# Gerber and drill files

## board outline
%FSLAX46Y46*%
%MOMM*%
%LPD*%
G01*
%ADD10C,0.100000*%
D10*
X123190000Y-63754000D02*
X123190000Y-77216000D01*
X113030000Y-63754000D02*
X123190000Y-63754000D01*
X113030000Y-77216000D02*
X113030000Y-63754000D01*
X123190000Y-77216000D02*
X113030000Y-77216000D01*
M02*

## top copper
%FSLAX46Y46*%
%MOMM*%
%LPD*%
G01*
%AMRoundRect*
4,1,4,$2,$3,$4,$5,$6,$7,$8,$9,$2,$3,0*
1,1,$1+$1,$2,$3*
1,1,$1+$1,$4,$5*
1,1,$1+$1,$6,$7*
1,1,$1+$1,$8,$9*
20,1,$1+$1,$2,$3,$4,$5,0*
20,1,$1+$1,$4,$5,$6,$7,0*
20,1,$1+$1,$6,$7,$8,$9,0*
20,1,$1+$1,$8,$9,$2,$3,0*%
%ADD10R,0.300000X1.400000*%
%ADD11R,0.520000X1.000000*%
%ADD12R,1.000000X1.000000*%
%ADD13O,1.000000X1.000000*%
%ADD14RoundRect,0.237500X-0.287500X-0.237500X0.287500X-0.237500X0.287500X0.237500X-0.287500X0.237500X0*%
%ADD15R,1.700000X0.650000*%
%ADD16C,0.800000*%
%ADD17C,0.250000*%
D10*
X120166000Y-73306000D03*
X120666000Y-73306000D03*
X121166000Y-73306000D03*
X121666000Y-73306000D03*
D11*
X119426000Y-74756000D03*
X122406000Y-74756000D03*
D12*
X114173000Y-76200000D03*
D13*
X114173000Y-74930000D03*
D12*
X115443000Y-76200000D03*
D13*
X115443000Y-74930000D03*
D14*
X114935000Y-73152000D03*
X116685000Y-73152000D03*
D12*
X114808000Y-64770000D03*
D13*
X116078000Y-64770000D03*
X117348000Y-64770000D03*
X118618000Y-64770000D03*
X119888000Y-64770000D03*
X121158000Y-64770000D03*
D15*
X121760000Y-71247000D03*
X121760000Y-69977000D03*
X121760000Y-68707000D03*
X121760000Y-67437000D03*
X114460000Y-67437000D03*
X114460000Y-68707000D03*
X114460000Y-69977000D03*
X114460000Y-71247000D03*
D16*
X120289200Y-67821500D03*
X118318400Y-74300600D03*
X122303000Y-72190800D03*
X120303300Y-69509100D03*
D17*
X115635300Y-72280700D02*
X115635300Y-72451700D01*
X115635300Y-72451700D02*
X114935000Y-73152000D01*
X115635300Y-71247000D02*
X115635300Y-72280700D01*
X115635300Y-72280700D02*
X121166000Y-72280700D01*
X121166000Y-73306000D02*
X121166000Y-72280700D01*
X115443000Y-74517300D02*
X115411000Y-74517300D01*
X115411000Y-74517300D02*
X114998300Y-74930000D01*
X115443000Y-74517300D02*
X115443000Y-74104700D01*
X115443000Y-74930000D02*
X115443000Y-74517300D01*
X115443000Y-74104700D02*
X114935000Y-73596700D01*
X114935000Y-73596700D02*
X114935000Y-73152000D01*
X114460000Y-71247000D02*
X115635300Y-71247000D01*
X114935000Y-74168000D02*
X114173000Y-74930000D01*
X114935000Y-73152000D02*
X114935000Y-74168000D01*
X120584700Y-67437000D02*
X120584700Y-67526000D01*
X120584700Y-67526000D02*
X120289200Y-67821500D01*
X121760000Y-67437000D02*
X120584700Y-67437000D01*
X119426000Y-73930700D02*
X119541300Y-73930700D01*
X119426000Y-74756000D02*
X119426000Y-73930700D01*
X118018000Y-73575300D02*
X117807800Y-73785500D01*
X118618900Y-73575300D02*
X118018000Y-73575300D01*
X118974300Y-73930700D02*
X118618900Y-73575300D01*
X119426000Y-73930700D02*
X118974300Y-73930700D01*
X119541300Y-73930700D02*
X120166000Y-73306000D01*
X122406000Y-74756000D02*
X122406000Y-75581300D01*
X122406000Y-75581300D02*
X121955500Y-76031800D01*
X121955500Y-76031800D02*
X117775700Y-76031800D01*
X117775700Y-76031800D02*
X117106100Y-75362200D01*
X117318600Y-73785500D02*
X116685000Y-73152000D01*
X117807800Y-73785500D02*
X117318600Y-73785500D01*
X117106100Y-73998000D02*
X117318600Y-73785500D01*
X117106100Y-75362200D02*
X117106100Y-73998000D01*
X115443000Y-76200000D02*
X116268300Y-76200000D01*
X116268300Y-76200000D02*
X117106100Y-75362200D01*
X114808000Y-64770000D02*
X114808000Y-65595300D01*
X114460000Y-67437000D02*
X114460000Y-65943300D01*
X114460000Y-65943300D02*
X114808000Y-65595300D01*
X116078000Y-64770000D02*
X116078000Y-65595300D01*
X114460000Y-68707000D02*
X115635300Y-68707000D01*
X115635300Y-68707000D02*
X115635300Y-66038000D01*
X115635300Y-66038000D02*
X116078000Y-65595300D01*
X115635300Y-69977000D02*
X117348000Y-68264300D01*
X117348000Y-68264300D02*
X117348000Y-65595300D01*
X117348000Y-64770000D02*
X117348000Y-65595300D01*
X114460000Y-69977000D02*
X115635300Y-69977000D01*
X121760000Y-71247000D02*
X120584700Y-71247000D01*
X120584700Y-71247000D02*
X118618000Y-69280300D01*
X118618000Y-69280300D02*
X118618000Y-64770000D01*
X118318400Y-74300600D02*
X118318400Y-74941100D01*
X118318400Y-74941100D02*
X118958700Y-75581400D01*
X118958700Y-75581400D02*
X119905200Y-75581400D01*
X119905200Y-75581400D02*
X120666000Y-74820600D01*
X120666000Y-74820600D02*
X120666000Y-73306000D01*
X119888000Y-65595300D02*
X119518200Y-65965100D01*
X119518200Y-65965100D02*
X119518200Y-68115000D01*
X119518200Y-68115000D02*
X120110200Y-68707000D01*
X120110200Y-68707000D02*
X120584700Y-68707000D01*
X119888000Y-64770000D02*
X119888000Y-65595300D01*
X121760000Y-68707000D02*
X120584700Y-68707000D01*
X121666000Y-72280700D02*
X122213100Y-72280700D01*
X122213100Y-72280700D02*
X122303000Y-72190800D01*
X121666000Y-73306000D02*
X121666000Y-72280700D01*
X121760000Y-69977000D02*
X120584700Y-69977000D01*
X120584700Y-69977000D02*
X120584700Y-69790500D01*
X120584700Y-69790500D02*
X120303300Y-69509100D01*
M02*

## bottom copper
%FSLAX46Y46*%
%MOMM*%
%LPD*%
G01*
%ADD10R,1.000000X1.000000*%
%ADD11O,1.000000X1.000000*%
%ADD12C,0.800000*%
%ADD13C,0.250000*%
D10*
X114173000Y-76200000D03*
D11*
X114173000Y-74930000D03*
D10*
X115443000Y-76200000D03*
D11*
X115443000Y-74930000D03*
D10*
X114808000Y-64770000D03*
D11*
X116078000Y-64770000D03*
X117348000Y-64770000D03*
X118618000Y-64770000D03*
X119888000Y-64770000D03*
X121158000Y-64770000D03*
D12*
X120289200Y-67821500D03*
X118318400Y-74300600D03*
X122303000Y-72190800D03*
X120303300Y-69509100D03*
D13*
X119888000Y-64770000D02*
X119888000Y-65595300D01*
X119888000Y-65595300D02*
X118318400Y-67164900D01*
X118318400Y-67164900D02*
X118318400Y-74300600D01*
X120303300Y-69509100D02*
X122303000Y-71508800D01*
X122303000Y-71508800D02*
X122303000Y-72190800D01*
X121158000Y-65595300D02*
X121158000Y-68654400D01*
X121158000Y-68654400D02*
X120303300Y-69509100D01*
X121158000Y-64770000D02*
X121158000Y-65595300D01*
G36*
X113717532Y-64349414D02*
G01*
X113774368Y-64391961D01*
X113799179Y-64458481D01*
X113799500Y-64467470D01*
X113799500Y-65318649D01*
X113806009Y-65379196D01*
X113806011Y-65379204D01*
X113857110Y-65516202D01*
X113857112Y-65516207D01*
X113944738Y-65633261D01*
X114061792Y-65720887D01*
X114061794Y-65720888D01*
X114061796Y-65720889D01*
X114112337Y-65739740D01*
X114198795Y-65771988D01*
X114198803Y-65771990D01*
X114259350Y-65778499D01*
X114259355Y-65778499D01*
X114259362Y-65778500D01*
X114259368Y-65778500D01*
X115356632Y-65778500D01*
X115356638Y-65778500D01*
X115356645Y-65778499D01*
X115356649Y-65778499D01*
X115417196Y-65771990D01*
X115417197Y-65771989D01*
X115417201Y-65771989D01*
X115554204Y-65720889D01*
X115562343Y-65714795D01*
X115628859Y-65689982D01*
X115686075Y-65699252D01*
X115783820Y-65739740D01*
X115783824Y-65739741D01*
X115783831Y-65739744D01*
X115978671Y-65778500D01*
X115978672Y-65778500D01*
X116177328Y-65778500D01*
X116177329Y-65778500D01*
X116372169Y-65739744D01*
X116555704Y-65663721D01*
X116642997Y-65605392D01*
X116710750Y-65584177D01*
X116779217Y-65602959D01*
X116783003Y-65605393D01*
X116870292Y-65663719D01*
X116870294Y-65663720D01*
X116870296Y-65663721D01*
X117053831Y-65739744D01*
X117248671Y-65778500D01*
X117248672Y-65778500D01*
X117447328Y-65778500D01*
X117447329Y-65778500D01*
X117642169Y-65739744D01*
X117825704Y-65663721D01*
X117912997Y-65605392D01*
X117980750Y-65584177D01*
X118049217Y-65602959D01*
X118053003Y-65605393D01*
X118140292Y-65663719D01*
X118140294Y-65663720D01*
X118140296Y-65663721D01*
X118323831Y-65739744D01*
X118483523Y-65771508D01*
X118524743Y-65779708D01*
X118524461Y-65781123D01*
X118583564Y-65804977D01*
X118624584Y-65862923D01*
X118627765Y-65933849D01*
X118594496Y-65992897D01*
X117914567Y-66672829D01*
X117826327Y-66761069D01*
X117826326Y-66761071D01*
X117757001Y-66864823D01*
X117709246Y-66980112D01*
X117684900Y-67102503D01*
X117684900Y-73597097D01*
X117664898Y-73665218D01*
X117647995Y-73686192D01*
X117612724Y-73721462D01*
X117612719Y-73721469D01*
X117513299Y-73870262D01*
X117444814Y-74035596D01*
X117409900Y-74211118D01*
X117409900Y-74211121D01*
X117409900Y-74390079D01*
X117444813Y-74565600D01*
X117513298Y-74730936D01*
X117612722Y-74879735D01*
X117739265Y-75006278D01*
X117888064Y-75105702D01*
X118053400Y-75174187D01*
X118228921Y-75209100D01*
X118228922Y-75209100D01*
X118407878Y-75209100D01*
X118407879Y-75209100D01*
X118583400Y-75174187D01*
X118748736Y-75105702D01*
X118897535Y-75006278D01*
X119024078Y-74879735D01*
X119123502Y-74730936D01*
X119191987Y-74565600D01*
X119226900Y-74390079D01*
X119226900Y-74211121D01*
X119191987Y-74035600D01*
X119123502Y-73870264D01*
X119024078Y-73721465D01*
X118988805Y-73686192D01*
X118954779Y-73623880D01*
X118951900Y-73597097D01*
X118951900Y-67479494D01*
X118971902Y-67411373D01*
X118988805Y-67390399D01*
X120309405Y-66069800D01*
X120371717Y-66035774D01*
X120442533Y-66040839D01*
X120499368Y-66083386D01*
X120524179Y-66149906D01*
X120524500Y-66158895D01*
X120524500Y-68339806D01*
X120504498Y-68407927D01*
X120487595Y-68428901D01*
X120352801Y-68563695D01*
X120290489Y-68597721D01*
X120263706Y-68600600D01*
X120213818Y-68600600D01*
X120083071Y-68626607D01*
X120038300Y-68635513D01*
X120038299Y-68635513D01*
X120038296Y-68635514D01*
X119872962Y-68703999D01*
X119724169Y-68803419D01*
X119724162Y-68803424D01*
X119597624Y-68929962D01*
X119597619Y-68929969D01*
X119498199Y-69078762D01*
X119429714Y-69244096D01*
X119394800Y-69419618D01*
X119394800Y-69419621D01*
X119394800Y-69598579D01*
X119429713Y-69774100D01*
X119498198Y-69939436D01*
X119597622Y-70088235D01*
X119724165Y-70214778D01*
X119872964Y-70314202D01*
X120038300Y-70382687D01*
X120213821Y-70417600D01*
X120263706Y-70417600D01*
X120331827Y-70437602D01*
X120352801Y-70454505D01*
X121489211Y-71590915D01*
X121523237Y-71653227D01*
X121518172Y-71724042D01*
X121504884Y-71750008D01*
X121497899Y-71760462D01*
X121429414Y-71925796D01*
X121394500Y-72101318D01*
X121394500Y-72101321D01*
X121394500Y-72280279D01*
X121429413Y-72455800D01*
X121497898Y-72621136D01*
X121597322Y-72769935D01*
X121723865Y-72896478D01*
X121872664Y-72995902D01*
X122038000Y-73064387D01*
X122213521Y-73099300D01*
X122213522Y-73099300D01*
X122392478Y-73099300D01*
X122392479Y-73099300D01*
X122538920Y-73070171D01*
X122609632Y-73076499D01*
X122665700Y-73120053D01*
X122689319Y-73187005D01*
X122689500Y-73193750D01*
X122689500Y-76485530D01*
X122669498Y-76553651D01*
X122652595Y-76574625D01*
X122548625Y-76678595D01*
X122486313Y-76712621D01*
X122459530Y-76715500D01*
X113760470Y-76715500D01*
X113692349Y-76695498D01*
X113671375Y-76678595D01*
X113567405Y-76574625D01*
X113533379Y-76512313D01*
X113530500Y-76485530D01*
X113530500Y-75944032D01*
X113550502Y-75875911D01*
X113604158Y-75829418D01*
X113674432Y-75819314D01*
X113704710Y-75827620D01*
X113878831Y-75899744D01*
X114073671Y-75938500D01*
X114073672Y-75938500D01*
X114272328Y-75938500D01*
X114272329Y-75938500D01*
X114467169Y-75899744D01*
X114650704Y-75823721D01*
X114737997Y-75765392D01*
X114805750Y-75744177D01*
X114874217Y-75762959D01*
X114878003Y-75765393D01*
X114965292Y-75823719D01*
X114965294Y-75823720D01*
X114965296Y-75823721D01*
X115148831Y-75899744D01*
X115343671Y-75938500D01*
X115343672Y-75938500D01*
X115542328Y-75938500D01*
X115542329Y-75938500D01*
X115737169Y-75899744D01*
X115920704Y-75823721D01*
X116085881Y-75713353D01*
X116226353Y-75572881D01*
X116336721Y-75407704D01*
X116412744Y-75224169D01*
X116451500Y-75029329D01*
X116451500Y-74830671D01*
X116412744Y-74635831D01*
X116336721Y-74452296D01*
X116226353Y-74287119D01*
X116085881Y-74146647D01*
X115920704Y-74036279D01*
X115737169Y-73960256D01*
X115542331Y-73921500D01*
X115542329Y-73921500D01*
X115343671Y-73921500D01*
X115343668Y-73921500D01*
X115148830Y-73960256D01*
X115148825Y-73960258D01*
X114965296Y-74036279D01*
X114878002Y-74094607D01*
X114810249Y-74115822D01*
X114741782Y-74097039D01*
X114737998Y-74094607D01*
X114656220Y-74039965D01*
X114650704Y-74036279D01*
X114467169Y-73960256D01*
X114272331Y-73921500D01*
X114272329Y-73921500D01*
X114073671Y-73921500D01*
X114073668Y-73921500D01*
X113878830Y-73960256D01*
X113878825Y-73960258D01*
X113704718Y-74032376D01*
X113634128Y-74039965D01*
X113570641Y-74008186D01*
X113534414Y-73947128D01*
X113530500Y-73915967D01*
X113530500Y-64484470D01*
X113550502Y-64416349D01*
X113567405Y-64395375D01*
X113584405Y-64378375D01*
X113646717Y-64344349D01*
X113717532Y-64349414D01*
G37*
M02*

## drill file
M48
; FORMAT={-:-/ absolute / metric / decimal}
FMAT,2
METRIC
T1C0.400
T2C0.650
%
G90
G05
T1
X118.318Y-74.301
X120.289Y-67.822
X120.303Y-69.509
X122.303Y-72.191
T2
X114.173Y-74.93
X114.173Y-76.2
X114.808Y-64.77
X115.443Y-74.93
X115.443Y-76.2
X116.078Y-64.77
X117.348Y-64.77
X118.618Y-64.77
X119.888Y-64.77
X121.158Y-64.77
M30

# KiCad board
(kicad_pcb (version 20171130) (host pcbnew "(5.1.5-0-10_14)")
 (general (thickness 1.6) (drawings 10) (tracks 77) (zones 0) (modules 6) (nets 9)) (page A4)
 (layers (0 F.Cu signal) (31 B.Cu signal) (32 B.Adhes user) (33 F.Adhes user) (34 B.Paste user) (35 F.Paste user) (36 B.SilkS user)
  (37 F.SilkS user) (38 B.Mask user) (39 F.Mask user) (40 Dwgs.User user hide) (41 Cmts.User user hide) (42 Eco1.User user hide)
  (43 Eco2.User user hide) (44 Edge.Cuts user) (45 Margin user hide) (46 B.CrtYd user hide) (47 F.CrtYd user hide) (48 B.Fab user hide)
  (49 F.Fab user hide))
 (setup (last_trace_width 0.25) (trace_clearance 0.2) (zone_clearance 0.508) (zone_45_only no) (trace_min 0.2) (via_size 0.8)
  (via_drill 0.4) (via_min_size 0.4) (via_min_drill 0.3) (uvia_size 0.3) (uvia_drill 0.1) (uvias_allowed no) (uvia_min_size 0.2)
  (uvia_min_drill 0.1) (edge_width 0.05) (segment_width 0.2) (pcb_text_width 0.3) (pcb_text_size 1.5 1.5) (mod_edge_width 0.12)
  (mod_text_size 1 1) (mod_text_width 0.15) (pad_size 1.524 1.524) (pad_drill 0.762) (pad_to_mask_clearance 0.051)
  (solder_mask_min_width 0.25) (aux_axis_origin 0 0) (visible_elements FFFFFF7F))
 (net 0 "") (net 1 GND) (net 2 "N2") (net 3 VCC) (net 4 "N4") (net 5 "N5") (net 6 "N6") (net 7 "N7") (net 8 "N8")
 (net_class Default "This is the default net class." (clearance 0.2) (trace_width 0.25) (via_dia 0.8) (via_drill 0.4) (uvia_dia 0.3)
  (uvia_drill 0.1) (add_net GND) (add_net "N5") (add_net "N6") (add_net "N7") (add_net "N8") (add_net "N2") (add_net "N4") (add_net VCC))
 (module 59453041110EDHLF (layer F.Cu) (at 120.916 73.406)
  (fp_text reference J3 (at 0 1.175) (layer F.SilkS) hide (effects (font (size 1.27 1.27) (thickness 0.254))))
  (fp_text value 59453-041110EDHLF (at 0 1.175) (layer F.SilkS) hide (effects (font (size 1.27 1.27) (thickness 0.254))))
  (pad 1 smd rect (at -0.75 -0.1) (size 0.3 1.4) (layers F.Cu F.Paste F.Mask) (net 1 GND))
  (pad 2 smd rect (at -0.25 -0.1) (size 0.3 1.4) (layers F.Cu F.Paste F.Mask) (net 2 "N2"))
  (pad 3 smd rect (at 0.25 -0.1) (size 0.3 1.4) (layers F.Cu F.Paste F.Mask) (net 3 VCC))
  (pad 4 smd rect (at 0.75 -0.1) (size 0.3 1.4) (layers F.Cu F.Paste F.Mask) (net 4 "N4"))
  (pad MP1 smd rect (at -1.49 1.35) (size 0.52 1) (layers F.Cu F.Paste F.Mask) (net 1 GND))
  (pad MP2 smd rect (at 1.49 1.35) (size 0.52 1) (layers F.Cu F.Paste F.Mask) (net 1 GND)))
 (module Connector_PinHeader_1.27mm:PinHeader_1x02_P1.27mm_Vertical (layer F.Cu) (at 114.173 76.2 180)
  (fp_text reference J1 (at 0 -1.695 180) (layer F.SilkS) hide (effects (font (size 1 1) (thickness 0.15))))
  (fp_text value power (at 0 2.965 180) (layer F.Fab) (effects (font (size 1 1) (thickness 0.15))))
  (pad 1 thru_hole rect (at 0 0 180) (size 1 1) (drill 0.65) (layers *.Cu *.Mask) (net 1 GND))
  (pad 2 thru_hole oval (at 0 1.27 180) (size 1 1) (drill 0.65) (layers *.Cu *.Mask) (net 3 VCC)))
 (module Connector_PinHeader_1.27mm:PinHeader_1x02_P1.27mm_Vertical (layer F.Cu) (at 115.443 76.2 180)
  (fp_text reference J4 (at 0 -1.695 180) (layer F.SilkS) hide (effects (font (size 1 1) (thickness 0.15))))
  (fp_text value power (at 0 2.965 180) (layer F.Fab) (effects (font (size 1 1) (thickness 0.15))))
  (pad 1 thru_hole rect (at 0 0 180) (size 1 1) (drill 0.65) (layers *.Cu *.Mask) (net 1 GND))
  (pad 2 thru_hole oval (at 0 1.27 180) (size 1 1) (drill 0.65) (layers *.Cu *.Mask) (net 3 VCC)))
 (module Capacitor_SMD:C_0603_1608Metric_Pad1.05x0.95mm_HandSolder (layer F.Cu) (at 115.81 73.152)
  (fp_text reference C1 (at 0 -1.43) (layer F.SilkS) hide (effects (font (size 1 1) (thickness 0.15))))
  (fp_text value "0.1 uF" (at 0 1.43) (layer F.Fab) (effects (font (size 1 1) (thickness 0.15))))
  (pad 1 smd roundrect (at -0.875 0) (size 1.05 0.95) (layers F.Cu F.Paste F.Mask) (roundrect_rratio 0.25) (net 3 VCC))
  (pad 2 smd roundrect (at 0.875 0) (size 1.05 0.95) (layers F.Cu F.Paste F.Mask) (roundrect_rratio 0.25) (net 1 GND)))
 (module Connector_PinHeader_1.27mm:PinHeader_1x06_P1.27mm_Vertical (layer F.Cu) (at 114.808 64.77 90)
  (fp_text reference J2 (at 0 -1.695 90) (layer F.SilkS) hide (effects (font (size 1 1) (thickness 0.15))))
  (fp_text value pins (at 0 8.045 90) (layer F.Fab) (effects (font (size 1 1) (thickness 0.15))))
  (pad 1 thru_hole rect (at 0 0 90) (size 1 1) (drill 0.65) (layers *.Cu *.Mask) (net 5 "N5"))
  (pad 2 thru_hole oval (at 0 1.27 90) (size 1 1) (drill 0.65) (layers *.Cu *.Mask) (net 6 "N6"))
  (pad 3 thru_hole oval (at 0 2.54 90) (size 1 1) (drill 0.65) (layers *.Cu *.Mask) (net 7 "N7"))
  (pad 4 thru_hole oval (at 0 3.81 90) (size 1 1) (drill 0.65) (layers *.Cu *.Mask) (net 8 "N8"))
  (pad 5 thru_hole oval (at 0 5.08 90) (size 1 1) (drill 0.65) (layers *.Cu *.Mask) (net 2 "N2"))
  (pad 6 thru_hole oval (at 0 6.35 90) (size 1 1) (drill 0.65) (layers *.Cu *.Mask) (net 4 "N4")))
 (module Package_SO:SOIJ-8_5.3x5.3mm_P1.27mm (layer F.Cu) (at 118.11 69.342 180)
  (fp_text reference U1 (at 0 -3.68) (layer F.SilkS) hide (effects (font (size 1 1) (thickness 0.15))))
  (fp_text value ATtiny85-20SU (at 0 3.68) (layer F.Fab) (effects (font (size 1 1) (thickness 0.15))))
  (pad 1 smd rect (at -3.65 -1.905 180) (size 1.7 0.65) (layers F.Cu F.Paste F.Mask) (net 8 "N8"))
  (pad 2 smd rect (at -3.65 -0.635 180) (size 1.7 0.65) (layers F.Cu F.Paste F.Mask) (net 4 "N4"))
  (pad 3 smd rect (at -3.65 0.635 180) (size 1.7 0.65) (layers F.Cu F.Paste F.Mask) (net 2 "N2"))
  (pad 4 smd rect (at -3.65 1.905 180) (size 1.7 0.65) (layers F.Cu F.Paste F.Mask) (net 1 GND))
  (pad 5 smd rect (at 3.65 1.905 180) (size 1.7 0.65) (layers F.Cu F.Paste F.Mask) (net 5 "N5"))
  (pad 6 smd rect (at 3.65 0.635 180) (size 1.7 0.65) (layers F.Cu F.Paste F.Mask) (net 6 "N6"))
  (pad 7 smd rect (at 3.65 -0.635 180) (size 1.7 0.65) (layers F.Cu F.Paste F.Mask) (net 7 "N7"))
  (pad 8 smd rect (at 3.65 -1.905 180) (size 1.7 0.65) (layers F.Cu F.Paste F.Mask) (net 3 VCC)))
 (gr_line (start 123.19 63.754) (end 123.19 77.216) (layer Edge.Cuts) (width 0.1))
 (gr_line (start 113.03 63.754) (end 123.19 63.754) (layer Edge.Cuts) (width 0.1))
 (gr_line (start 113.03 77.216) (end 113.03 63.754) (layer Edge.Cuts) (width 0.1))
 (gr_line (start 123.19 77.216) (end 113.03 77.216) (layer Edge.Cuts) (width 0.1))
 (segment (start 115.6353 72.2807) (end 115.6353 72.4517) (width 0.25) (layer F.Cu) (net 3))
 (segment (start 115.6353 72.4517) (end 114.935 73.152) (width 0.25) (layer F.Cu) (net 3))
 (segment (start 115.6353 71.247) (end 115.6353 72.2807) (width 0.25) (layer F.Cu) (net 3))
 (segment (start 115.6353 72.2807) (end 121.166 72.2807) (width 0.25) (layer F.Cu) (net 3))
 (segment (start 121.166 73.306) (end 121.166 72.2807) (width 0.25) (layer F.Cu) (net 3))
 (segment (start 115.443 74.5173) (end 115.411 74.5173) (width 0.25) (layer F.Cu) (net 3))
 (segment (start 115.411 74.5173) (end 114.9983 74.93) (width 0.25) (layer F.Cu) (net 3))
 (segment (start 115.443 74.5173) (end 115.443 74.1047) (width 0.25) (layer F.Cu) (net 3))
 (segment (start 115.443 74.93) (end 115.443 74.5173) (width 0.25) (layer F.Cu) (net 3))
 (segment (start 115.443 74.1047) (end 114.935 73.5967) (width 0.25) (layer F.Cu) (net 3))
 (segment (start 114.935 73.5967) (end 114.935 73.152) (width 0.25) (layer F.Cu) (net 3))
 (segment (start 114.46 71.247) (end 115.6353 71.247) (width 0.25) (layer F.Cu) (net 3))
 (segment (start 114.935 74.168) (end 114.173 74.93) (width 0.25) (layer F.Cu) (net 3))
 (segment (start 114.935 73.152) (end 114.935 74.168) (width 0.25) (layer F.Cu) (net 3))
 (segment (start 120.5847 67.437) (end 120.5847 67.526) (width 0.25) (layer F.Cu) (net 1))
 (segment (start 120.5847 67.526) (end 120.2892 67.8215) (width 0.25) (layer F.Cu) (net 1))
 (segment (start 121.76 67.437) (end 120.5847 67.437) (width 0.25) (layer F.Cu) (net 1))
 (via (at 120.2892 67.8215) (size 0.8) (layers F.Cu B.Cu) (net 1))
 (segment (start 119.426 73.9307) (end 119.5413 73.9307) (width 0.25) (layer F.Cu) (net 1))
 (segment (start 119.426 74.756) (end 119.426 73.9307) (width 0.25) (layer F.Cu) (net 1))
 (segment (start 118.018 73.5753) (end 117.8078 73.7855) (width 0.25) (layer F.Cu) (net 1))
 (segment (start 118.6189 73.5753) (end 118.018 73.5753) (width 0.25) (layer F.Cu) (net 1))
 (segment (start 118.9743 73.9307) (end 118.6189 73.5753) (width 0.25) (layer F.Cu) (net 1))
 (segment (start 119.426 73.9307) (end 118.9743 73.9307) (width 0.25) (layer F.Cu) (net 1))
 (segment (start 119.5413 73.9307) (end 120.166 73.306) (width 0.25) (layer F.Cu) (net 1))
 (segment (start 122.406 74.756) (end 122.406 75.5813) (width 0.25) (layer F.Cu) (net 1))
 (segment (start 122.406 75.5813) (end 121.9555 76.0318) (width 0.25) (layer F.Cu) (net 1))
 (segment (start 121.9555 76.0318) (end 117.7757 76.0318) (width 0.25) (layer F.Cu) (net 1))
 (segment (start 117.7757 76.0318) (end 117.1061 75.3622) (width 0.25) (layer F.Cu) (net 1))
 (segment (start 117.3186 73.7855) (end 116.685 73.152) (width 0.25) (layer F.Cu) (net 1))
 (segment (start 117.8078 73.7855) (end 117.3186 73.7855) (width 0.25) (layer F.Cu) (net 1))
 (segment (start 117.1061 73.998) (end 117.3186 73.7855) (width 0.25) (layer F.Cu) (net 1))
 (segment (start 117.1061 75.3622) (end 117.1061 73.998) (width 0.25) (layer F.Cu) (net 1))
 (segment (start 115.443 76.2) (end 116.2683 76.2) (width 0.25) (layer F.Cu) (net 1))
 (segment (start 116.2683 76.2) (end 117.1061 75.3622) (width 0.25) (layer F.Cu) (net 1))
 (segment (start 114.808 64.77) (end 114.808 65.5953) (width 0.25) (layer F.Cu) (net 5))
 (segment (start 114.46 67.437) (end 114.46 65.9433) (width 0.25) (layer F.Cu) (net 5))
 (segment (start 114.46 65.9433) (end 114.808 65.5953) (width 0.25) (layer F.Cu) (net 5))
 (segment (start 116.078 64.77) (end 116.078 65.5953) (width 0.25) (layer F.Cu) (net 6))
 (segment (start 114.46 68.707) (end 115.6353 68.707) (width 0.25) (layer F.Cu) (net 6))
 (segment (start 115.6353 68.707) (end 115.6353 66.038) (width 0.25) (layer F.Cu) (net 6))
 (segment (start 115.6353 66.038) (end 116.078 65.5953) (width 0.25) (layer F.Cu) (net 6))
 (segment (start 115.6353 69.977) (end 117.348 68.2643) (width 0.25) (layer F.Cu) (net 7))
 (segment (start 117.348 68.2643) (end 117.348 65.5953) (width 0.25) (layer F.Cu) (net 7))
 (segment (start 117.348 64.77) (end 117.348 65.5953) (width 0.25) (layer F.Cu) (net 7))
 (segment (start 114.46 69.977) (end 115.6353 69.977) (width 0.25) (layer F.Cu) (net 7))
 (segment (start 121.76 71.247) (end 120.5847 71.247) (width 0.25) (layer F.Cu) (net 8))
 (segment (start 120.5847 71.247) (end 118.618 69.2803) (width 0.25) (layer F.Cu) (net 8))
 (segment (start 118.618 69.2803) (end 118.618 64.77) (width 0.25) (layer F.Cu) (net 8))
 (segment (start 119.888 64.77) (end 119.888 65.5953) (width 0.25) (layer B.Cu) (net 2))
 (segment (start 118.3184 74.3006) (end 118.3184 74.9411) (width 0.25) (layer F.Cu) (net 2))
 (segment (start 118.3184 74.9411) (end 118.9587 75.5814) (width 0.25) (layer F.Cu) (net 2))
 (segment (start 118.9587 75.5814) (end 119.9052 75.5814) (width 0.25) (layer F.Cu) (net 2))
 (segment (start 119.9052 75.5814) (end 120.666 74.8206) (width 0.25) (layer F.Cu) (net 2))
 (segment (start 120.666 74.8206) (end 120.666 73.306) (width 0.25) (layer F.Cu) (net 2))
 (segment (start 119.888 65.5953) (end 118.3184 67.1649) (width 0.25) (layer B.Cu) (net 2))
 (segment (start 118.3184 67.1649) (end 118.3184 74.3006) (width 0.25) (layer B.Cu) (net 2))
 (segment (start 119.888 65.5953) (end 119.5182 65.9651) (width 0.25) (layer F.Cu) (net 2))
 (segment (start 119.5182 65.9651) (end 119.5182 68.115) (width 0.25) (layer F.Cu) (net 2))
 (segment (start 119.5182 68.115) (end 120.1102 68.707) (width 0.25) (layer F.Cu) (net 2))
 (segment (start 120.1102 68.707) (end 120.5847 68.707) (width 0.25) (layer F.Cu) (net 2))
 (segment (start 119.888 64.77) (end 119.888 65.5953) (width 0.25) (layer F.Cu) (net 2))
 (segment (start 121.76 68.707) (end 120.5847 68.707) (width 0.25) (layer F.Cu) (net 2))
 (via (at 118.3184 74.3006) (size 0.8) (layers F.Cu B.Cu) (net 2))
 (segment (start 120.3033 69.5091) (end 122.303 71.5088) (width 0.25) (layer B.Cu) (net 4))
 (segment (start 122.303 71.5088) (end 122.303 72.1908) (width 0.25) (layer B.Cu) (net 4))
 (segment (start 121.666 72.2807) (end 122.2131 72.2807) (width 0.25) (layer F.Cu) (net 4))
 (segment (start 122.2131 72.2807) (end 122.303 72.1908) (width 0.25) (layer F.Cu) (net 4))
 (segment (start 121.666 73.306) (end 121.666 72.2807) (width 0.25) (layer F.Cu) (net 4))
 (segment (start 121.158 65.5953) (end 121.158 68.6544) (width 0.25) (layer B.Cu) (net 4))
 (segment (start 121.158 68.6544) (end 120.3033 69.5091) (width 0.25) (layer B.Cu) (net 4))
 (segment (start 121.158 64.77) (end 121.158 65.5953) (width 0.25) (layer B.Cu) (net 4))
 (segment (start 121.76 69.977) (end 120.5847 69.977) (width 0.25) (layer F.Cu) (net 4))
 (segment (start 120.5847 69.977) (end 120.5847 69.7905) (width 0.25) (layer F.Cu) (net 4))
 (segment (start 120.5847 69.7905) (end 120.3033 69.5091) (width 0.25) (layer F.Cu) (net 4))
 (via (at 122.303 72.1908) (size 0.8) (layers F.Cu B.Cu) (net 4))
 (via (at 120.3033 69.5091) (size 0.8) (layers F.Cu B.Cu) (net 4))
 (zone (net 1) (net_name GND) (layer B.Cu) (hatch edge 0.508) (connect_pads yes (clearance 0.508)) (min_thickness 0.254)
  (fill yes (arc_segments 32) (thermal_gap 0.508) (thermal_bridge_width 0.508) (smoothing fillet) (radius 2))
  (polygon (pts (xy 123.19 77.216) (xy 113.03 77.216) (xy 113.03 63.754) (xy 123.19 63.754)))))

